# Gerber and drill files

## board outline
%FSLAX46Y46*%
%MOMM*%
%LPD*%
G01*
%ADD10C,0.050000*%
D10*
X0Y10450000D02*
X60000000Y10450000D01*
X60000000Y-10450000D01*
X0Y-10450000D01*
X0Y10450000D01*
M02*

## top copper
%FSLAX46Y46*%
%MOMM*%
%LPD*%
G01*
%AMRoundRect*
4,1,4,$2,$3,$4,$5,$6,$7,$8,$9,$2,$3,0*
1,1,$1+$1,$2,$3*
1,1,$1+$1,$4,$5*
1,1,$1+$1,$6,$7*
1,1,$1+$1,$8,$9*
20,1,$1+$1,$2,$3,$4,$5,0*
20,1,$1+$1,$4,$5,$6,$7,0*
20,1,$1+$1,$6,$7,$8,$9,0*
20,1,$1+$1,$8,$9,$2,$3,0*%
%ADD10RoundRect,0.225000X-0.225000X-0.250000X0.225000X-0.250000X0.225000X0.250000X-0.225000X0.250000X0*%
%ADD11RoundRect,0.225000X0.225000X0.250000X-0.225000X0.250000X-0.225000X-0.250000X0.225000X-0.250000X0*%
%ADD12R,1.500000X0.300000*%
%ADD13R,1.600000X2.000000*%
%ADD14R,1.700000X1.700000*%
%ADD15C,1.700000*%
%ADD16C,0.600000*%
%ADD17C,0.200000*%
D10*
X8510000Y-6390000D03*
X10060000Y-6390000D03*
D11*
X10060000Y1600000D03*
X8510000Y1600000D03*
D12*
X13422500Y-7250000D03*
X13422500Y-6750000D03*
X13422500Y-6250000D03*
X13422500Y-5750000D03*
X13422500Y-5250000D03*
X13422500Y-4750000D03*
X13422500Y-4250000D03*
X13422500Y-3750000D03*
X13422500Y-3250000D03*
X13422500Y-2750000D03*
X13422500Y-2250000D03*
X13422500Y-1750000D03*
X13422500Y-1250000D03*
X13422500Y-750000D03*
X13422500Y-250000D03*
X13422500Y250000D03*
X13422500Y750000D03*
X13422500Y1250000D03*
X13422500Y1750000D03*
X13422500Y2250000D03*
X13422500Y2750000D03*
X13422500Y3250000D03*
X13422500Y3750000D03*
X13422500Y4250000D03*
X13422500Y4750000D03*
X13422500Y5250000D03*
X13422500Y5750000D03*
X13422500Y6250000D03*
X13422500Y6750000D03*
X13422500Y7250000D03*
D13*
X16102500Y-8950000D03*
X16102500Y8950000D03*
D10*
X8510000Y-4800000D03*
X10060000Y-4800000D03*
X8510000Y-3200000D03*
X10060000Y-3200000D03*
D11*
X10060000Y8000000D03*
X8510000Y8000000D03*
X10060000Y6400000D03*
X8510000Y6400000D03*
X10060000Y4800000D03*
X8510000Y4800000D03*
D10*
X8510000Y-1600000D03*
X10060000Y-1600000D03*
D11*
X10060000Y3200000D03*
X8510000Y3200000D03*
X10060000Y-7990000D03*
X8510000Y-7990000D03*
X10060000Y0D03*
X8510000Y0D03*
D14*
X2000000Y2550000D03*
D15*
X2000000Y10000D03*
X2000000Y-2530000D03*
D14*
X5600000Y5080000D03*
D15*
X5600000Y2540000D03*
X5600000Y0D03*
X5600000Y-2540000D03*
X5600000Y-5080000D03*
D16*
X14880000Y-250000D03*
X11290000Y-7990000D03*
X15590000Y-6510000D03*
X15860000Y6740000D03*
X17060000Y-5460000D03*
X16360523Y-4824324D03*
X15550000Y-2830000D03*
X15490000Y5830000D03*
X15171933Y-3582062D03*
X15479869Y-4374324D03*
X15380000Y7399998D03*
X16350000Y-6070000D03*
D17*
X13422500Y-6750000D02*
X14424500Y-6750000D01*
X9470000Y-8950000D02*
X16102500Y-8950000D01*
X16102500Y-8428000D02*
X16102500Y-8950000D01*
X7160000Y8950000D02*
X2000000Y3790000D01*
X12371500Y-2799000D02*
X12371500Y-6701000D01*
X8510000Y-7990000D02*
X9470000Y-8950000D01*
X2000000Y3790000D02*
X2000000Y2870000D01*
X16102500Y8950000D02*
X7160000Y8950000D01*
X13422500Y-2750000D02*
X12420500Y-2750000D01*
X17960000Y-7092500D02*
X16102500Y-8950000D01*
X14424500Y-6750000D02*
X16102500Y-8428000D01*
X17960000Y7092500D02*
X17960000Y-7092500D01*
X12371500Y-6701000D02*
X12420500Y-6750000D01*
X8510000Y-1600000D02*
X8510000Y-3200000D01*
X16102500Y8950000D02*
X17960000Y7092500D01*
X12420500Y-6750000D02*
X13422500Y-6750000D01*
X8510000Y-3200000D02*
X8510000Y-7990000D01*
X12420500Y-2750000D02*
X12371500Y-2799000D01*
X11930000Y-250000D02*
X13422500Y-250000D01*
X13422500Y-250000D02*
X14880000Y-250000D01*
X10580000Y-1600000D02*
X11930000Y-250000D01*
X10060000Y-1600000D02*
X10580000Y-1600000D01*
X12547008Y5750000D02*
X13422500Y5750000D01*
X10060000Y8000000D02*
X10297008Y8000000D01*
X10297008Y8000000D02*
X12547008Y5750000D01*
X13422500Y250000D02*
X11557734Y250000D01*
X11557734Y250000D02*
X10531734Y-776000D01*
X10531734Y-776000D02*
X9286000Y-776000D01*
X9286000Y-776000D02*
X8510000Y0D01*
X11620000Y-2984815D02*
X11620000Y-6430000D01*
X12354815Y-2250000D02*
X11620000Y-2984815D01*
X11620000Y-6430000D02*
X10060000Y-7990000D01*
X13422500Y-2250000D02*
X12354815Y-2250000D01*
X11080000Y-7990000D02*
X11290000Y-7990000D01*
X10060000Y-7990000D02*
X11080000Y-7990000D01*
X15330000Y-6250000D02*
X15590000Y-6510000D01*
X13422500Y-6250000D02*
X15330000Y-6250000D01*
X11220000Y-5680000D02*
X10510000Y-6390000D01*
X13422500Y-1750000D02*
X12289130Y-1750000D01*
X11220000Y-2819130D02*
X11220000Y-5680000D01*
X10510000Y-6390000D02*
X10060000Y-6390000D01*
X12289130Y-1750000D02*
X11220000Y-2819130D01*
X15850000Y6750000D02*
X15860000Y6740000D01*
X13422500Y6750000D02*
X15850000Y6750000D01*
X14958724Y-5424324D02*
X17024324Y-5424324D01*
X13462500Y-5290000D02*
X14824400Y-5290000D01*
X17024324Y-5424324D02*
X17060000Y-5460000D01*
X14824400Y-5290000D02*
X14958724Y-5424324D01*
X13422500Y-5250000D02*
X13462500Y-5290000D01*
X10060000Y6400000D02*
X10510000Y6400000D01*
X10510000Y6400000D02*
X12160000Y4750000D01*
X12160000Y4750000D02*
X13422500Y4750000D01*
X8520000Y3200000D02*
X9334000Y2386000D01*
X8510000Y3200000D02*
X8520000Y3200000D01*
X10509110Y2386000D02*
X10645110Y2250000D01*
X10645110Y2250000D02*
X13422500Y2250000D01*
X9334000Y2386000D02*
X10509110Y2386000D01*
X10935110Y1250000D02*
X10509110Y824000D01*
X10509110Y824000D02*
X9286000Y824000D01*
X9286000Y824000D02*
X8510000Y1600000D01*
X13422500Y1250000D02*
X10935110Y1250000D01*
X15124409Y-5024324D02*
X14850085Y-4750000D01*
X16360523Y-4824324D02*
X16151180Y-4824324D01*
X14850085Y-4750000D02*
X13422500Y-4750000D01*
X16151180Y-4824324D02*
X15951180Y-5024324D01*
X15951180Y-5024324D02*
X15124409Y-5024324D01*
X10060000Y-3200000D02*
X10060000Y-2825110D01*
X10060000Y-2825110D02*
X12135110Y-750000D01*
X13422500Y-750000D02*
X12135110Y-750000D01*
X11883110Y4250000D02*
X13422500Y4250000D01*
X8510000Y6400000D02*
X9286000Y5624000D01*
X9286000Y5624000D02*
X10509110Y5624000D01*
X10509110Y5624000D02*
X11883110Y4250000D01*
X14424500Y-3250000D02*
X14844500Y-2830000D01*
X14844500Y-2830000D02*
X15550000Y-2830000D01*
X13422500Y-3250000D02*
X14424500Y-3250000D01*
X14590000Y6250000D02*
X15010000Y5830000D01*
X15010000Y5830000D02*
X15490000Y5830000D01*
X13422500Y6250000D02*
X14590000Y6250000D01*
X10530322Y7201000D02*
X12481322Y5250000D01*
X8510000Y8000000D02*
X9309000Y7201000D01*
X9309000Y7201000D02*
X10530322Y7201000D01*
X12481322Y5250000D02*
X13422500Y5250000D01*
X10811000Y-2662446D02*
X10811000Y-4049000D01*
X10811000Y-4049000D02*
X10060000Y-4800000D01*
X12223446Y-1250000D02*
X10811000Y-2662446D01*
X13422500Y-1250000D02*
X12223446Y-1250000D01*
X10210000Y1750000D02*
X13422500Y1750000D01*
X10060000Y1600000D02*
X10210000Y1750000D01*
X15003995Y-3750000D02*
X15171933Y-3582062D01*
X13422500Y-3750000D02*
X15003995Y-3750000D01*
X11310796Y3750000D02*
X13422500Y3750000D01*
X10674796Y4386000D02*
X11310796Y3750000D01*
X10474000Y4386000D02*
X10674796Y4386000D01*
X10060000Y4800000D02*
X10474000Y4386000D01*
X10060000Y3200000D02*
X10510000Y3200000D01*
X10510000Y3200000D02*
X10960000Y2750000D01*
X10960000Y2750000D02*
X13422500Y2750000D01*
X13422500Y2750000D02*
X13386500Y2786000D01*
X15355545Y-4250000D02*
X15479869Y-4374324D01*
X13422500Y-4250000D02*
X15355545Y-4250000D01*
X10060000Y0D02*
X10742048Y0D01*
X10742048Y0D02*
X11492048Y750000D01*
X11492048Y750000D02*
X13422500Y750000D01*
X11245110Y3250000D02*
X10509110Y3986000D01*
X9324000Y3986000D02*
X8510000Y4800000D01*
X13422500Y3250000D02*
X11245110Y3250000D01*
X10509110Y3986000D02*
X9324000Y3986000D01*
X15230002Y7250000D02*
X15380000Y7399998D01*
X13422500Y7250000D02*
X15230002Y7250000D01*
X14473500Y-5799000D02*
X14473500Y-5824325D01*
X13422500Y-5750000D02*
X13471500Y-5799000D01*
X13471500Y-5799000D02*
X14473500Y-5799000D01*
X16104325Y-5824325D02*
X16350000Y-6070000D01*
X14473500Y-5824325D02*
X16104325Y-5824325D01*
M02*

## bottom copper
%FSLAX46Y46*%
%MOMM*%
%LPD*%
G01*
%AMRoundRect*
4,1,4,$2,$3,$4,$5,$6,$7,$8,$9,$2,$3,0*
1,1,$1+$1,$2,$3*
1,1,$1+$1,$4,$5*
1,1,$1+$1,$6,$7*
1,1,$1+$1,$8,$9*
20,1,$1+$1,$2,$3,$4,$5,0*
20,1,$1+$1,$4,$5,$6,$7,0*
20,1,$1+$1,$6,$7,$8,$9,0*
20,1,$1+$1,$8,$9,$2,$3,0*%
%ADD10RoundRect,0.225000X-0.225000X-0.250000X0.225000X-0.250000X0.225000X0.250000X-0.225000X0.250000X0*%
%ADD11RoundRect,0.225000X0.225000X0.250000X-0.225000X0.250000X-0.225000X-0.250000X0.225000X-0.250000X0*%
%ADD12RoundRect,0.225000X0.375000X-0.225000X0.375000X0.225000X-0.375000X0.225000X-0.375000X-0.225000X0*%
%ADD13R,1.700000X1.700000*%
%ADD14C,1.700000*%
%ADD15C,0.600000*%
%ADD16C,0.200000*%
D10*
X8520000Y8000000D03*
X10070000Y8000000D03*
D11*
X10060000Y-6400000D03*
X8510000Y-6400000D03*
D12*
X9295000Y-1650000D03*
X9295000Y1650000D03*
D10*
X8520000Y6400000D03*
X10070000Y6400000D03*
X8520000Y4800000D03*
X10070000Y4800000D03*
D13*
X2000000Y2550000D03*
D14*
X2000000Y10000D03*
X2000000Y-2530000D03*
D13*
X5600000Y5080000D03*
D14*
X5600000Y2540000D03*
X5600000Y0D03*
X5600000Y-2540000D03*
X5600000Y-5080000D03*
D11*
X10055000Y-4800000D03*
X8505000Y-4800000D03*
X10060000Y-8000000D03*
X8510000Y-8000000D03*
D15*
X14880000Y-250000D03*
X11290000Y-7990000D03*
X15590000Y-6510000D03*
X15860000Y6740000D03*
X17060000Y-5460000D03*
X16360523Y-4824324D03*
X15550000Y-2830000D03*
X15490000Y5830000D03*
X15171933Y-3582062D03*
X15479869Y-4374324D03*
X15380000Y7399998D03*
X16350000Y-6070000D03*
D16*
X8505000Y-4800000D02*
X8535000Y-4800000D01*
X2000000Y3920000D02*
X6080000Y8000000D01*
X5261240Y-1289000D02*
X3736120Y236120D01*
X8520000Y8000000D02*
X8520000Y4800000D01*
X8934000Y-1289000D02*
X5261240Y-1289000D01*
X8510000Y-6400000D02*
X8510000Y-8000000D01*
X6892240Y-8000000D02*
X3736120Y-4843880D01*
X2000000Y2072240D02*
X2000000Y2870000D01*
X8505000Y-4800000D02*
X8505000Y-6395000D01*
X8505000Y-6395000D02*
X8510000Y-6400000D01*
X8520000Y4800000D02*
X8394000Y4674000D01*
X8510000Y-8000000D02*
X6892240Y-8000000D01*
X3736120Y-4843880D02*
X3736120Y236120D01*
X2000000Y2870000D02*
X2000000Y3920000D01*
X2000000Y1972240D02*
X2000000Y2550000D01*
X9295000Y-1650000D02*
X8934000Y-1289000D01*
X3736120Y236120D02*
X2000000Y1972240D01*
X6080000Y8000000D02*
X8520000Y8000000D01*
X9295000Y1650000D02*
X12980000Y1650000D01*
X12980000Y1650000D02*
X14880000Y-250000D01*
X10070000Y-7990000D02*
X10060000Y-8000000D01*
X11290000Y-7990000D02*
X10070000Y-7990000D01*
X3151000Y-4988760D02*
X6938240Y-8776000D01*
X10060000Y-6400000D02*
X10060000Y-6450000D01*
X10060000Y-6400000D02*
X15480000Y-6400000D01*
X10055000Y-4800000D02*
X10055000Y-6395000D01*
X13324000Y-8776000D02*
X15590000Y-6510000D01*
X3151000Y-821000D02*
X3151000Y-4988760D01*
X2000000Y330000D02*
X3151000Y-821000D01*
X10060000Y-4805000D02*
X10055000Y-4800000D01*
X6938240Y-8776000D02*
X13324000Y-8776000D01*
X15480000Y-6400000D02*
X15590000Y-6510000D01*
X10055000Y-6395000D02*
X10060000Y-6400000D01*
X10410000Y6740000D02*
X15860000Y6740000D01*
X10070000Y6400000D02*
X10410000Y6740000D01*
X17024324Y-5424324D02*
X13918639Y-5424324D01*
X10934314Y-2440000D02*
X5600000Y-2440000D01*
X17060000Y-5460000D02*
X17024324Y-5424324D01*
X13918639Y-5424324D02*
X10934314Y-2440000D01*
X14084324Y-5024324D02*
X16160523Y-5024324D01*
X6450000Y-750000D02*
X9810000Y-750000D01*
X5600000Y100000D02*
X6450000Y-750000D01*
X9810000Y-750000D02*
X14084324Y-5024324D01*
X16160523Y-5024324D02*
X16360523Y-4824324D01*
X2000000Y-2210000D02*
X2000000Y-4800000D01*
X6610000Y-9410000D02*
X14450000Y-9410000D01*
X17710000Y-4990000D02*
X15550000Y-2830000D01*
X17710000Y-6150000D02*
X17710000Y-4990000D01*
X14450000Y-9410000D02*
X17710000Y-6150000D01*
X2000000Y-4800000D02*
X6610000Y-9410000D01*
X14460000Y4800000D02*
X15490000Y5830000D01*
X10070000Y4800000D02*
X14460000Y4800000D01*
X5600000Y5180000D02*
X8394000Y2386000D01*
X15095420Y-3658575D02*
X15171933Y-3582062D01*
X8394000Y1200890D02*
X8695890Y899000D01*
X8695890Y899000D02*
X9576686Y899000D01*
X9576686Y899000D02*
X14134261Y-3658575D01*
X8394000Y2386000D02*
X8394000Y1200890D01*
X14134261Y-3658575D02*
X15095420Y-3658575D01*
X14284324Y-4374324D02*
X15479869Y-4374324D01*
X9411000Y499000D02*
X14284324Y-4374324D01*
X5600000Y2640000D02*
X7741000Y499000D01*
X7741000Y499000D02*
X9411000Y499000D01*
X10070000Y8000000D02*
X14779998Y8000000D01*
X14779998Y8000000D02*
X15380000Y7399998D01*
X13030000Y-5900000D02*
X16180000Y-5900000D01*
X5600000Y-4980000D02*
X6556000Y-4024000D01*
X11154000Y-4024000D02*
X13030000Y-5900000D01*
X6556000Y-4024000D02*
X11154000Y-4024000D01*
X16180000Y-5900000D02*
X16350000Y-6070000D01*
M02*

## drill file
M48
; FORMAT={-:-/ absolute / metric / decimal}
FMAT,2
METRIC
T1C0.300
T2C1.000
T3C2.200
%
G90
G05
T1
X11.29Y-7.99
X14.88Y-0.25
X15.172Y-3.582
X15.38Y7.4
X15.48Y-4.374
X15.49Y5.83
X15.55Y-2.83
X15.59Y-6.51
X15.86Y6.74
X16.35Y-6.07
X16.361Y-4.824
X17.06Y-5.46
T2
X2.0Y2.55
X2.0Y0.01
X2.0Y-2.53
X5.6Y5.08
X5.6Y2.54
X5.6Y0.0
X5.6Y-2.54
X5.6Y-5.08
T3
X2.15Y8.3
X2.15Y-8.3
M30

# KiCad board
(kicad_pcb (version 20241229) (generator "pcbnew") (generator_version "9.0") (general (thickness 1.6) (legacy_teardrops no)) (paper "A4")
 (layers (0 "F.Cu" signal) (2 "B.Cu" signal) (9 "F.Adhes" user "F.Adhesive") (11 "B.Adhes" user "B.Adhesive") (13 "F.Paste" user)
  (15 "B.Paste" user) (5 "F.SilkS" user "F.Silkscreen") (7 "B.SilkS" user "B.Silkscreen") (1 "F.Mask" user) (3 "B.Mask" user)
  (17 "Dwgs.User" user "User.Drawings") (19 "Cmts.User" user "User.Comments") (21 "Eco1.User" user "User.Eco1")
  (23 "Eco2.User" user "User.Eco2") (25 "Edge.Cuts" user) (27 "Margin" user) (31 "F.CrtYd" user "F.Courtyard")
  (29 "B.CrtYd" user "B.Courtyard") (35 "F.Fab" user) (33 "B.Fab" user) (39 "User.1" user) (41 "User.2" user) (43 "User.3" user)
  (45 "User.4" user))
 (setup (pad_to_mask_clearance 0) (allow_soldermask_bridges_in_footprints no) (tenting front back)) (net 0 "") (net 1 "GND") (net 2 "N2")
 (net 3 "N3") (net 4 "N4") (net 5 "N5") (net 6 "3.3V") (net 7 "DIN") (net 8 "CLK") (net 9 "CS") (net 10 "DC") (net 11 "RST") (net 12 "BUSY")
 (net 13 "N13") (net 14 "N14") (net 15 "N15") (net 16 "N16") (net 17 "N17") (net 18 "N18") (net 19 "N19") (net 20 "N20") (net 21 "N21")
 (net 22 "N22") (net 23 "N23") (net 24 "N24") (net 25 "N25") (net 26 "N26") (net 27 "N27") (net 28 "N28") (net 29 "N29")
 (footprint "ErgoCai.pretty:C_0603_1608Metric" (layer "F.Cu") (at 9.285 6.39)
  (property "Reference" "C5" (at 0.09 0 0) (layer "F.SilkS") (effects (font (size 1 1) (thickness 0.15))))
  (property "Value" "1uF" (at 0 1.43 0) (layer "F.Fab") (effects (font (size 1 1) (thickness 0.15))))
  (pad "1" smd roundrect (at -0.775 0) (size 0.9 0.95) (layers "F.Cu" "F.Mask" "F.Paste") (roundrect_rratio 0.25) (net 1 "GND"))
  (pad "2" smd roundrect (at 0.775 0) (size 0.9 0.95) (layers "F.Cu" "F.Mask" "F.Paste") (roundrect_rratio 0.25) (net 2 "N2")))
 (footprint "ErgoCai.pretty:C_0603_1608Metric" (layer "F.Cu") (at 9.285 -1.6 180)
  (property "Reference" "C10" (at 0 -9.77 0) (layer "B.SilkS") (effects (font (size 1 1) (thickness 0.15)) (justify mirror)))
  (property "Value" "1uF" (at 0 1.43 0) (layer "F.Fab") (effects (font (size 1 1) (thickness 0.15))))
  (pad "1" smd roundrect (at -0.775 0 180) (size 0.9 0.95) (layers "F.Cu" "F.Mask" "F.Paste") (roundrect_rratio 0.25) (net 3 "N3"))
  (pad "2" smd roundrect (at 0.775 0 180) (size 0.9 0.95) (layers "F.Cu" "F.Mask" "F.Paste") (roundrect_rratio 0.25) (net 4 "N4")))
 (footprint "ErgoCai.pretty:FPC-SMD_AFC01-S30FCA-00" (layer "F.Cu") (at 14.7625 0 90)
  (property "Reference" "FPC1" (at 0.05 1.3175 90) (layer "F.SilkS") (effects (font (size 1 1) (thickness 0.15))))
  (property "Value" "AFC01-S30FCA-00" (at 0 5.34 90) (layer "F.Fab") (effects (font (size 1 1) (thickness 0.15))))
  (pad "1" smd rect (at -7.25 -1.34 90) (size 0.3 1.5) (layers "F.Cu" "F.Mask" "F.Paste") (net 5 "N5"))
  (pad "2" smd rect (at -6.75 -1.34 90) (size 0.3 1.5) (layers "F.Cu" "F.Mask" "F.Paste") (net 1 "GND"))
  (pad "3" smd rect (at -6.25 -1.34 90) (size 0.3 1.5) (layers "F.Cu" "F.Mask" "F.Paste") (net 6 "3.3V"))
  (pad "4" smd rect (at -5.75 -1.34 90) (size 0.3 1.5) (layers "F.Cu" "F.Mask" "F.Paste") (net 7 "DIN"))
  (pad "5" smd rect (at -5.25 -1.34 90) (size 0.3 1.5) (layers "F.Cu" "F.Mask" "F.Paste") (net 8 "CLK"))
  (pad "6" smd rect (at -4.75 -1.34 90) (size 0.3 1.5) (layers "F.Cu" "F.Mask" "F.Paste") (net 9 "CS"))
  (pad "7" smd rect (at -4.25 -1.34 90) (size 0.3 1.5) (layers "F.Cu" "F.Mask" "F.Paste") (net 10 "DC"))
  (pad "8" smd rect (at -3.75 -1.34 90) (size 0.3 1.5) (layers "F.Cu" "F.Mask" "F.Paste") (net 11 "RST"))
  (pad "9" smd rect (at -3.25 -1.34 90) (size 0.3 1.5) (layers "F.Cu" "F.Mask" "F.Paste") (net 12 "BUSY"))
  (pad "10" smd rect (at -2.75 -1.34 90) (size 0.3 1.5) (layers "F.Cu" "F.Mask" "F.Paste") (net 1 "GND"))
  (pad "11" smd rect (at -2.25 -1.34 90) (size 0.3 1.5) (layers "F.Cu" "F.Mask" "F.Paste") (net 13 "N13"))
  (pad "12" smd rect (at -1.75 -1.34 90) (size 0.3 1.5) (layers "F.Cu" "F.Mask" "F.Paste") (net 2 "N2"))
  (pad "13" smd rect (at -1.25 -1.34 90) (size 0.3 1.5) (layers "F.Cu" "F.Mask" "F.Paste") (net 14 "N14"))
  (pad "14" smd rect (at -0.75 -1.34 90) (size 0.3 1.5) (layers "F.Cu" "F.Mask" "F.Paste") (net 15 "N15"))
  (pad "15" smd rect (at -0.25 -1.34 90) (size 0.3 1.5) (layers "F.Cu" "F.Mask" "F.Paste") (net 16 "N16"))
  (pad "16" smd rect (at 0.25 -1.34 90) (size 0.3 1.5) (layers "F.Cu" "F.Mask" "F.Paste") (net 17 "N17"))
  (pad "17" smd rect (at 0.75 -1.34 90) (size 0.3 1.5) (layers "F.Cu" "F.Mask" "F.Paste") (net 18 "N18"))
  (pad "18" smd rect (at 1.25 -1.34 90) (size 0.3 1.5) (layers "F.Cu" "F.Mask" "F.Paste") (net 4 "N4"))
  (pad "19" smd rect (at 1.75 -1.34 90) (size 0.3 1.5) (layers "F.Cu" "F.Mask" "F.Paste") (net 3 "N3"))
  (pad "20" smd rect (at 2.25 -1.34 90) (size 0.3 1.5) (layers "F.Cu" "F.Mask" "F.Paste") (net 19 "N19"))
  (pad "21" smd rect (at 2.75 -1.34 90) (size 0.3 1.5) (layers "F.Cu" "F.Mask" "F.Paste") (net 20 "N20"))
  (pad "22" smd rect (at 3.25 -1.34 90) (size 0.3 1.5) (layers "F.Cu" "F.Mask" "F.Paste") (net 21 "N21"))
  (pad "23" smd rect (at 3.75 -1.34 90) (size 0.3 1.5) (layers "F.Cu" "F.Mask" "F.Paste") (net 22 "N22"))
  (pad "24" smd rect (at 4.25 -1.34 90) (size 0.3 1.5) (layers "F.Cu" "F.Mask" "F.Paste") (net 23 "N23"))
  (pad "25" smd rect (at 4.75 -1.34 90) (size 0.3 1.5) (layers "F.Cu" "F.Mask" "F.Paste") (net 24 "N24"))
  (pad "26" smd rect (at 5.25 -1.34 90) (size 0.3 1.5) (layers "F.Cu" "F.Mask" "F.Paste") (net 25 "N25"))
  (pad "27" smd rect (at 5.75 -1.34 90) (size 0.3 1.5) (layers "F.Cu" "F.Mask" "F.Paste") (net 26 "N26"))
  (pad "28" smd rect (at 6.25 -1.34 90) (size 0.3 1.5) (layers "F.Cu" "F.Mask" "F.Paste") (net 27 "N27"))
  (pad "29" smd rect (at 6.75 -1.34 90) (size 0.3 1.5) (layers "F.Cu" "F.Mask" "F.Paste") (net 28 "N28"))
  (pad "30" smd rect (at 7.25 -1.34 90) (size 0.3 1.5) (layers "F.Cu" "F.Mask" "F.Paste") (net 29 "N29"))
  (pad "31" smd rect (at -8.95 1.34 90) (size 2 1.6) (layers "F.Cu" "F.Mask" "F.Paste") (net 1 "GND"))
  (pad "32" smd rect (at 8.95 1.34 270) (size 2 1.6) (layers "F.Cu" "F.Mask" "F.Paste") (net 1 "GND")))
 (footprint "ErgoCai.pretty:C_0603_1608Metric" (layer "F.Cu") (at 9.285 4.8)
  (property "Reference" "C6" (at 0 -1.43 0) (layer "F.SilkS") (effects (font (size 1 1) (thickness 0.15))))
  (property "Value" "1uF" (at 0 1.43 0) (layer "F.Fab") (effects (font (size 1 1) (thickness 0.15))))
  (pad "1" smd roundrect (at -0.775 0) (size 0.9 0.95) (layers "F.Cu" "F.Mask" "F.Paste") (roundrect_rratio 0.25) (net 1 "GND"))
  (pad "2" smd roundrect (at 0.775 0) (size 0.9 0.95) (layers "F.Cu" "F.Mask" "F.Paste") (roundrect_rratio 0.25) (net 14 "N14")))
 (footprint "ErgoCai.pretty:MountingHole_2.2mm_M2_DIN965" (layer "F.Cu") (at 2.15 -8.3)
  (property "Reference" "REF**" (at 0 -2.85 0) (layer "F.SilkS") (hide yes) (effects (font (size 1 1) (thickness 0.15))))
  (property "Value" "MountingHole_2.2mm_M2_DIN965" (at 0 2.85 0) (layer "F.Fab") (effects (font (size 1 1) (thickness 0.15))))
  (pad "" np_thru_hole circle (at 0 0) (size 2.2 2.2) (drill 2.2) (layers "*.Cu" "*.Mask")))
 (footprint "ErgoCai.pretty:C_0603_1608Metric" (layer "F.Cu") (at 9.285 3.2)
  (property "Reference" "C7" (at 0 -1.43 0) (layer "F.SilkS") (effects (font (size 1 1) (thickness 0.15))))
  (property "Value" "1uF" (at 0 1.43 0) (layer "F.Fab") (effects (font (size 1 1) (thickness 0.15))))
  (pad "1" smd roundrect (at -0.775 0) (size 0.9 0.95) (layers "F.Cu" "F.Mask" "F.Paste") (roundrect_rratio 0.25) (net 1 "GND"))
  (pad "2" smd roundrect (at 0.775 0) (size 0.9 0.95) (layers "F.Cu" "F.Mask" "F.Paste") (roundrect_rratio 0.25) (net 15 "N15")))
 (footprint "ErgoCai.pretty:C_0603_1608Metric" (layer "F.Cu") (at 9.285 -8 180)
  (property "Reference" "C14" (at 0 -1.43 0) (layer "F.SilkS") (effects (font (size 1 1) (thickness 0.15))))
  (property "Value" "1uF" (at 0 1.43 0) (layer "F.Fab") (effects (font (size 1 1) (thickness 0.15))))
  (pad "1" smd roundrect (at -0.775 0 180) (size 0.9 0.95) (layers "F.Cu" "F.Mask" "F.Paste") (roundrect_rratio 0.25) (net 26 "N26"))
  (pad "2" smd roundrect (at 0.775 0 180) (size 0.9 0.95) (layers "F.Cu" "F.Mask" "F.Paste") (roundrect_rratio 0.25) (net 25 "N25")))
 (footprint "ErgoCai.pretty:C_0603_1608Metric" (layer "F.Cu") (at 9.285 -6.4 180)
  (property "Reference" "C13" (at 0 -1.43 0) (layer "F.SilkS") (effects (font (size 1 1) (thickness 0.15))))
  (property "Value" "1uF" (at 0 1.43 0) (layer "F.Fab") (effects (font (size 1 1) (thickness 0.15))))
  (pad "1" smd roundrect (at -0.775 0 180) (size 0.9 0.95) (layers "F.Cu" "F.Mask" "F.Paste") (roundrect_rratio 0.25) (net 24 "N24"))
  (pad "2" smd roundrect (at 0.775 0 180) (size 0.9 0.95) (layers "F.Cu" "F.Mask" "F.Paste") (roundrect_rratio 0.25) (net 23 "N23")))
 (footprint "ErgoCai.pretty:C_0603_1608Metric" (layer "F.Cu") (at 9.285 -4.8 180)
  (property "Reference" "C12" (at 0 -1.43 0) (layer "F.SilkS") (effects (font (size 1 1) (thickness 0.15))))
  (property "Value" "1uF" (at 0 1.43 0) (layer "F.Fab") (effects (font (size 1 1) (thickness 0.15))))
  (pad "1" smd roundrect (at -0.775 0 180) (size 0.9 0.95) (layers "F.Cu" "F.Mask" "F.Paste") (roundrect_rratio 0.25) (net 22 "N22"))
  (pad "2" smd roundrect (at 0.775 0 180) (size 0.9 0.95) (layers "F.Cu" "F.Mask" "F.Paste") (roundrect_rratio 0.25) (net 21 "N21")))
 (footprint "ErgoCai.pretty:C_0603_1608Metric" (layer "F.Cu") (at 9.285 1.6)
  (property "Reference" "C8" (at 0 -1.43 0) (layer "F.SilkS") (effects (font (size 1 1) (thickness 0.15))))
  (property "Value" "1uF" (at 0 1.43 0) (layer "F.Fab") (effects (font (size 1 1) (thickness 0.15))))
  (pad "1" smd roundrect (at -0.775 0) (size 0.9 0.95) (layers "F.Cu" "F.Mask" "F.Paste") (roundrect_rratio 0.25) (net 1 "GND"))
  (pad "2" smd roundrect (at 0.775 0) (size 0.9 0.95) (layers "F.Cu" "F.Mask" "F.Paste") (roundrect_rratio 0.25) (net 16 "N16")))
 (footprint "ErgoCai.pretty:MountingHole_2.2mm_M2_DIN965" (layer "F.Cu") (at 2.15 8.3)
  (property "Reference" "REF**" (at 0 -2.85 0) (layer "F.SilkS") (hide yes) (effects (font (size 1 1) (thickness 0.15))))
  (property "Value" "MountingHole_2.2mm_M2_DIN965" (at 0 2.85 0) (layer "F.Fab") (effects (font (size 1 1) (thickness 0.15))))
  (pad "" np_thru_hole circle (at 0 0) (size 2.2 2.2) (drill 2.2) (layers "*.Cu" "*.Mask")))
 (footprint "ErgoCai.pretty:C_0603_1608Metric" (layer "F.Cu") (at 9.285 -3.2 180)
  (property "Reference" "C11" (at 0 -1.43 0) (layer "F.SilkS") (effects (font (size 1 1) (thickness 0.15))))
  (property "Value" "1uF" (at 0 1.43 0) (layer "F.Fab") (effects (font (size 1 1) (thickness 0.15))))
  (pad "1" smd roundrect (at -0.775 0 180) (size 0.9 0.95) (layers "F.Cu" "F.Mask" "F.Paste") (roundrect_rratio 0.25) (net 20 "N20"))
  (pad "2" smd roundrect (at 0.775 0 180) (size 0.9 0.95) (layers "F.Cu" "F.Mask" "F.Paste") (roundrect_rratio 0.25) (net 19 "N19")))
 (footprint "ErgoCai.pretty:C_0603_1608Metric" (layer "F.Cu") (at 9.285 7.99 180)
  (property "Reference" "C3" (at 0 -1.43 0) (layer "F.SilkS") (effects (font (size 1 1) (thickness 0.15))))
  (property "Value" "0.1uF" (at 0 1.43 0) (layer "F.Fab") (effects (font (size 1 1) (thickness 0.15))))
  (pad "1" smd roundrect (at -0.775 0 180) (size 0.9 0.95) (layers "F.Cu" "F.Mask" "F.Paste") (roundrect_rratio 0.25) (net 13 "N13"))
  (pad "2" smd roundrect (at 0.775 0 180) (size 0.9 0.95) (layers "F.Cu" "F.Mask" "F.Paste") (roundrect_rratio 0.25) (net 1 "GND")))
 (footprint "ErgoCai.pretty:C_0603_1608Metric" (layer "F.Cu") (at 9.285 0 180)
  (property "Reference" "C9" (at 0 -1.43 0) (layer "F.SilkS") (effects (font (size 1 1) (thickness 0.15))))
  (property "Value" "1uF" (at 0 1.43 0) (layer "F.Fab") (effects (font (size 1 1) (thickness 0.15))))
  (pad "1" smd roundrect (at -0.775 0 180) (size 0.9 0.95) (layers "F.Cu" "F.Mask" "F.Paste") (roundrect_rratio 0.25) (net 18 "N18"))
  (pad "2" smd roundrect (at 0.775 0 180) (size 0.9 0.95) (layers "F.Cu" "F.Mask" "F.Paste") (roundrect_rratio 0.25) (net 17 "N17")))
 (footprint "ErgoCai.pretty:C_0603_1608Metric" (layer "B.Cu") (at 9.295 -8)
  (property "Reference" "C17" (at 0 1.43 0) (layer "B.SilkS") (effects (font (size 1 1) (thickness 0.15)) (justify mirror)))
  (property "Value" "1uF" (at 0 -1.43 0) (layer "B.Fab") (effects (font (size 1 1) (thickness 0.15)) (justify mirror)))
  (pad "1" smd roundrect (at -0.775 0) (size 0.9 0.95) (layers "B.Cu" "B.Mask" "B.Paste") (roundrect_rratio 0.25) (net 1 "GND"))
  (pad "2" smd roundrect (at 0.775 0) (size 0.9 0.95) (layers "B.Cu" "B.Mask" "B.Paste") (roundrect_rratio 0.25) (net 29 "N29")))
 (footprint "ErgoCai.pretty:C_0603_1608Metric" (layer "B.Cu") (at 9.285 6.4 180)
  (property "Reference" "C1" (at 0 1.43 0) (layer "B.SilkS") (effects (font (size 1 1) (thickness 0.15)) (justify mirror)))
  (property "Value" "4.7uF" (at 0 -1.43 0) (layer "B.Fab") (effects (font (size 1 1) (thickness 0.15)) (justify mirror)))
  (pad "1" smd roundrect (at -0.775 0 180) (size 0.9 0.95) (layers "B.Cu" "B.Mask" "B.Paste") (roundrect_rratio 0.25) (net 6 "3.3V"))
  (pad "2" smd roundrect (at 0.775 0 180) (size 0.9 0.95) (layers "B.Cu" "B.Mask" "B.Paste") (roundrect_rratio 0.25) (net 1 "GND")))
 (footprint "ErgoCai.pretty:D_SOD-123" (layer "B.Cu") (at 9.295 0 90)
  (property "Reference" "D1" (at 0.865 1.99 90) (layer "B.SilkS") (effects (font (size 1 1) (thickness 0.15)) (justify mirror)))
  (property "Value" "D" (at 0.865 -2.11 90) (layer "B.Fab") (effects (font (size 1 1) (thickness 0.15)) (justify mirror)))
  (pad "1" smd roundrect (at -1.65 0 90) (size 0.9 1.2) (layers "B.Cu" "B.Mask" "B.Paste") (roundrect_rratio 0.25) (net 1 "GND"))
  (pad "2" smd roundrect (at 1.65 0 90) (size 0.9 1.2) (layers "B.Cu" "B.Mask" "B.Paste") (roundrect_rratio 0.25) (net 16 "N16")))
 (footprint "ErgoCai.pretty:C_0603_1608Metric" (layer "B.Cu") (at 9.295 -6.4)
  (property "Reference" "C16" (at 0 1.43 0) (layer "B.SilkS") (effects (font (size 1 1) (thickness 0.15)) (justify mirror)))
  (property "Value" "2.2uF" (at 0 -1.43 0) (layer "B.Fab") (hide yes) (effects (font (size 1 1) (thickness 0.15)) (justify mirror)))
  (pad "1" smd roundrect (at -0.775 0) (size 0.9 0.95) (layers "B.Cu" "B.Mask" "B.Paste") (roundrect_rratio 0.25) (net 1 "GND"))
  (pad "2" smd roundrect (at 0.775 0) (size 0.9 0.95) (layers "B.Cu" "B.Mask" "B.Paste") (roundrect_rratio 0.25) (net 28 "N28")))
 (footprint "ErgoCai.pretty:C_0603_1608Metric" (layer "B.Cu") (at 9.295 -4.8)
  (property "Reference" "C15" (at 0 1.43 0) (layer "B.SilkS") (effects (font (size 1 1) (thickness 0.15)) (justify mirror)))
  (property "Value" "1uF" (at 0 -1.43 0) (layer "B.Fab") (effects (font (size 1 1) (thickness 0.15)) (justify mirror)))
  (pad "1" smd roundrect (at -0.775 0) (size 0.9 0.95) (layers "B.Cu" "B.Mask" "B.Paste") (roundrect_rratio 0.25) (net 1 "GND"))
  (pad "2" smd roundrect (at 0.775 0) (size 0.9 0.95) (layers "B.Cu" "B.Mask" "B.Paste") (roundrect_rratio 0.25) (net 27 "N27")))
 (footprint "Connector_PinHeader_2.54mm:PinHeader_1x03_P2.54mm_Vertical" (layer "B.Cu") (at 2 -2.55 180)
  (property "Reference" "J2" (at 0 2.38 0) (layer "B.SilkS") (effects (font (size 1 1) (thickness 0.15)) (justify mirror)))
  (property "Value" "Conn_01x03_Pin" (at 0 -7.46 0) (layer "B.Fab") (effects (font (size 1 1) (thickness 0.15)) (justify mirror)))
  (pad "1" thru_hole rect (at 0 0 180) (size 1.7 1.7) (drill 1) (layers "*.Cu" "*.Mask") (remove_unused_layers no) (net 1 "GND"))
  (pad "2" thru_hole circle (at 0 -2.54 180) (size 1.7 1.7) (drill 1) (layers "*.Cu" "*.Mask") (remove_unused_layers no) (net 6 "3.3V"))
  (pad "3" thru_hole circle (at 0 -5.08 180) (size 1.7 1.7) (drill 1) (layers "*.Cu" "*.Mask") (remove_unused_layers no) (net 12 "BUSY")))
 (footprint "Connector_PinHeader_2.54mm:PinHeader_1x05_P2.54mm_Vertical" (layer "B.Cu") (at 5.6 -5.08 180)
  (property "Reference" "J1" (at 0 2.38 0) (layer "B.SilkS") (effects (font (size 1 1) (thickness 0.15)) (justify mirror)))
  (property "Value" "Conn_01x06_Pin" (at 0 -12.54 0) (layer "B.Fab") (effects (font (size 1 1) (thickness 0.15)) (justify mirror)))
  (pad "1" thru_hole rect (at 0 0 180) (size 1.7 1.7) (drill 1) (layers "*.Cu" "*.Mask") (remove_unused_layers no) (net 11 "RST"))
  (pad "2" thru_hole circle (at 0 -2.54 180) (size 1.7 1.7) (drill 1) (layers "*.Cu" "*.Mask") (remove_unused_layers no) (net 10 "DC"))
  (pad "3" thru_hole circle (at 0 -5.08 180) (size 1.7 1.7) (drill 1) (layers "*.Cu" "*.Mask") (remove_unused_layers no) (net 9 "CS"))
  (pad "4" thru_hole circle (at 0 -7.62 180) (size 1.7 1.7) (drill 1) (layers "*.Cu" "*.Mask") (remove_unused_layers no) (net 8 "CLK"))
  (pad "5" thru_hole circle (at 0 -10.16 180) (size 1.7 1.7) (drill 1) (layers "*.Cu" "*.Mask") (remove_unused_layers no) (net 7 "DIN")))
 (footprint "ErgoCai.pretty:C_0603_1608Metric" (layer "B.Cu") (at 9.28 4.8 180)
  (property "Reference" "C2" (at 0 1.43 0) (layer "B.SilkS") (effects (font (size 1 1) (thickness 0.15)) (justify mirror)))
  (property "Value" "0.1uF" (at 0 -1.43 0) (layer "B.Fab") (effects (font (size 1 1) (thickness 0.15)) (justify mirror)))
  (pad "1" smd roundrect (at -0.775 0 180) (size 0.9 0.95) (layers "B.Cu" "B.Mask" "B.Paste") (roundrect_rratio 0.25) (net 6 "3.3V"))
  (pad "2" smd roundrect (at 0.775 0 180) (size 0.9 0.95) (layers "B.Cu" "B.Mask" "B.Paste") (roundrect_rratio 0.25) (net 1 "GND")))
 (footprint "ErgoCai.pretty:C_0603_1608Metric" (layer "B.Cu") (at 9.285 8 180)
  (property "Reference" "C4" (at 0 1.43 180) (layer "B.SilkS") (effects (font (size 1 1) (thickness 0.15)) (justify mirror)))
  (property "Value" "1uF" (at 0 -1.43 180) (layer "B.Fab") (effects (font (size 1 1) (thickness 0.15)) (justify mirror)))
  (pad "1" smd roundrect (at -0.775 0 180) (size 0.9 0.95) (layers "B.Cu" "B.Mask" "B.Paste") (roundrect_rratio 0.25) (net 13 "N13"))
  (pad "2" smd roundrect (at 0.775 0 180) (size 0.9 0.95) (layers "B.Cu" "B.Mask" "B.Paste") (roundrect_rratio 0.25) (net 1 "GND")))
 (gr_rect (start 0 -10.45) (end 60 10.45) (stroke (width 0.05) (type solid)) (fill no) (layer "Edge.Cuts"))
 (segment (start 13.4225 6.75) (end 14.4245 6.75) (width 0.2) (layer "F.Cu") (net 1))
 (segment (start 9.47 8.95) (end 16.1025 8.95) (width 0.2) (layer "F.Cu") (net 1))
 (segment (start 16.1025 8.428) (end 16.1025 8.95) (width 0.2) (layer "F.Cu") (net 1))
 (segment (start 7.16 -8.95) (end 2 -3.79) (width 0.2) (layer "F.Cu") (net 1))
 (segment (start 12.3715 2.799) (end 12.3715 6.701) (width 0.2) (layer "F.Cu") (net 1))
 (segment (start 8.51 7.99) (end 9.47 8.95) (width 0.2) (layer "F.Cu") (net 1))
 (segment (start 2 -3.79) (end 2 -2.87) (width 0.2) (layer "F.Cu") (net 1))
 (segment (start 16.1025 -8.95) (end 7.16 -8.95) (width 0.2) (layer "F.Cu") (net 1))
 (segment (start 13.4225 2.75) (end 12.4205 2.75) (width 0.2) (layer "F.Cu") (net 1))
 (segment (start 17.96 7.0925) (end 16.1025 8.95) (width 0.2) (layer "F.Cu") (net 1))
 (segment (start 14.4245 6.75) (end 16.1025 8.428) (width 0.2) (layer "F.Cu") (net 1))
 (segment (start 17.96 -7.0925) (end 17.96 7.0925) (width 0.2) (layer "F.Cu") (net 1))
 (segment (start 12.3715 6.701) (end 12.4205 6.75) (width 0.2) (layer "F.Cu") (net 1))
 (segment (start 8.51 1.6) (end 8.51 3.2) (width 0.2) (layer "F.Cu") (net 1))
 (segment (start 16.1025 -8.95) (end 17.96 -7.0925) (width 0.2) (layer "F.Cu") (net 1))
 (segment (start 12.4205 6.75) (end 13.4225 6.75) (width 0.2) (layer "F.Cu") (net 1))
 (segment (start 8.51 3.2) (end 8.51 7.99) (width 0.2) (layer "F.Cu") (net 1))
 (segment (start 12.4205 2.75) (end 12.3715 2.799) (width 0.2) (layer "F.Cu") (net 1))
 (segment (start 8.505 4.8) (end 8.535 4.8) (width 0.2) (layer "B.Cu") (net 1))
 (segment (start 2 -3.92) (end 6.08 -8) (width 0.2) (layer "B.Cu") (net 1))
 (segment (start 5.26124 1.289) (end 3.73612 -0.23612) (width 0.2) (layer "B.Cu") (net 1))
 (segment (start 8.52 -8) (end 8.52 -4.8) (width 0.2) (layer "B.Cu") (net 1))
 (segment (start 8.934 1.289) (end 5.26124 1.289) (width 0.2) (layer "B.Cu") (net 1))
 (segment (start 8.51 6.4) (end 8.51 8) (width 0.2) (layer "B.Cu") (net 1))
 (segment (start 6.89224 8) (end 3.73612 4.84388) (width 0.2) (layer "B.Cu") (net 1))
 (segment (start 2 -2.07224) (end 2 -2.87) (width 0.2) (layer "B.Cu") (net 1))
 (segment (start 8.505 4.8) (end 8.505 6.395) (width 0.2) (layer "B.Cu") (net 1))
 (segment (start 8.505 6.395) (end 8.51 6.4) (width 0.2) (layer "B.Cu") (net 1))
 (segment (start 8.52 -4.8) (end 8.394 -4.674) (width 0.2) (layer "B.Cu") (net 1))
 (segment (start 8.51 8) (end 6.89224 8) (width 0.2) (layer "B.Cu") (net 1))
 (segment (start 3.73612 4.84388) (end 3.73612 -0.23612) (width 0.2) (layer "B.Cu") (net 1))
 (segment (start 2 -2.87) (end 2 -3.92) (width 0.2) (layer "B.Cu") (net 1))
 (segment (start 2 -1.97224) (end 2 -2.55) (width 0.2) (layer "B.Cu") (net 1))
 (segment (start 9.295 1.65) (end 8.934 1.289) (width 0.2) (layer "B.Cu") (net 1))
 (segment (start 3.73612 -0.23612) (end 2 -1.97224) (width 0.2) (layer "B.Cu") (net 1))
 (segment (start 6.08 -8) (end 8.52 -8) (width 0.2) (layer "B.Cu") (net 1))
 (segment (start 11.93 0.25) (end 13.4225 0.25) (width 0.2) (layer "F.Cu") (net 16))
 (segment (start 13.4225 0.25) (end 14.88 0.25) (width 0.2) (layer "F.Cu") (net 16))
 (segment (start 10.58 1.6) (end 11.93 0.25) (width 0.2) (layer "F.Cu") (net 16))
 (segment (start 10.06 1.6) (end 10.58 1.6) (width 0.2) (layer "F.Cu") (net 16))
 (via (at 14.88 0.25) (size 0.6) (drill 0.3) (layers "F.Cu" "B.Cu") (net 16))
 (segment (start 9.295 -1.65) (end 12.98 -1.65) (width 0.2) (layer "B.Cu") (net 16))
 (segment (start 12.98 -1.65) (end 14.88 0.25) (width 0.2) (layer "B.Cu") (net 16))
 (segment (start 12.547008 -5.75) (end 13.4225 -5.75) (width 0.2) (layer "F.Cu") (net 26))
 (segment (start 10.06 -8) (end 10.297008 -8) (width 0.2) (layer "F.Cu") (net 26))
 (segment (start 10.297008 -8) (end 12.547008 -5.75) (width 0.2) (layer "F.Cu") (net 26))
 (segment (start 13.4225 -0.25) (end 11.557734 -0.25) (width 0.2) (layer "F.Cu") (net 17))
 (segment (start 11.557734 -0.25) (end 10.531734 0.776) (width 0.2) (layer "F.Cu") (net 17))
 (segment (start 10.531734 0.776) (end 9.286 0.776) (width 0.2) (layer "F.Cu") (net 17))
 (segment (start 9.286 0.776) (end 8.51 0) (width 0.2) (layer "F.Cu") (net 17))
 (segment (start 11.62 2.984815) (end 11.62 6.43) (width 0.2) (layer "F.Cu") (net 13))
 (segment (start 12.354815 2.25) (end 11.62 2.984815) (width 0.2) (layer "F.Cu") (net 13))
 (segment (start 11.62 6.43) (end 10.06 7.99) (width 0.2) (layer "F.Cu") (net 13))
 (segment (start 13.4225 2.25) (end 12.354815 2.25) (width 0.2) (layer "F.Cu") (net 13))
 (segment (start 11.08 7.99) (end 11.29 7.99) (width 0.2) (layer "F.Cu") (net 13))
 (segment (start 10.06 7.99) (end 11.08 7.99) (width 0.2) (layer "F.Cu") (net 13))
 (via (at 11.29 7.99) (size 0.6) (drill 0.3) (layers "F.Cu" "B.Cu") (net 13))
 (segment (start 10.07 7.99) (end 10.06 8) (width 0.2) (layer "B.Cu") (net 13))
 (segment (start 11.29 7.99) (end 10.07 7.99) (width 0.2) (layer "B.Cu") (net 13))
 (segment (start 15.33 6.25) (end 15.59 6.51) (width 0.2) (layer "F.Cu") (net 6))
 (segment (start 13.4225 6.25) (end 15.33 6.25) (width 0.2) (layer "F.Cu") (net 6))
 (via (at 15.59 6.51) (size 0.6) (drill 0.3) (layers "F.Cu" "B.Cu") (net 6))
 (segment (start 3.151 4.98876) (end 6.93824 8.776) (width 0.2) (layer "B.Cu") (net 6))
 (segment (start 10.06 6.4) (end 10.06 6.45) (width 0.2) (layer "B.Cu") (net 6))
 (segment (start 10.06 6.4) (end 15.48 6.4) (width 0.2) (layer "B.Cu") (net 6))
 (segment (start 10.055 4.8) (end 10.055 6.395) (width 0.2) (layer "B.Cu") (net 6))
 (segment (start 13.324 8.776) (end 15.59 6.51) (width 0.2) (layer "B.Cu") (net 6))
 (segment (start 3.151 0.821) (end 3.151 4.98876) (width 0.2) (layer "B.Cu") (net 6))
 (segment (start 2 -0.33) (end 3.151 0.821) (width 0.2) (layer "B.Cu") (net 6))
 (segment (start 10.06 4.805) (end 10.055 4.8) (width 0.2) (layer "B.Cu") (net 6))
 (segment (start 6.93824 8.776) (end 13.324 8.776) (width 0.2) (layer "B.Cu") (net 6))
 (segment (start 15.48 6.4) (end 15.59 6.51) (width 0.2) (layer "B.Cu") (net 6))
 (segment (start 10.055 6.395) (end 10.06 6.4) (width 0.2) (layer "B.Cu") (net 6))
 (segment (start 11.22 5.68) (end 10.51 6.39) (width 0.2) (layer "F.Cu") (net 2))
 (segment (start 13.4225 1.75) (end 12.28913 1.75) (width 0.2) (layer "F.Cu") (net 2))
 (segment (start 11.22 2.81913) (end 11.22 5.68) (width 0.2) (layer "F.Cu") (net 2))
 (segment (start 10.51 6.39) (end 10.06 6.39) (width 0.2) (layer "F.Cu") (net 2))
 (segment (start 12.28913 1.75) (end 11.22 2.81913) (width 0.2) (layer "F.Cu") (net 2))
 (segment (start 15.85 -6.75) (end 15.86 -6.74) (width 0.2) (layer "F.Cu") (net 28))
 (segment (start 13.4225 -6.75) (end 15.85 -6.75) (width 0.2) (layer "F.Cu") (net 28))
 (via (at 15.86 -6.74) (size 0.6) (drill 0.3) (layers "F.Cu" "B.Cu") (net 28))
 (segment (start 10.41 -6.74) (end 15.86 -6.74) (width 0.2) (layer "B.Cu") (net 28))
 (segment (start 10.07 -6.4) (end 10.41 -6.74) (width 0.2) (layer "B.Cu") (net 28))
 (segment (start 14.958724 5.424324) (end 17.024324 5.424324) (width 0.2) (layer "F.Cu") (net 8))
 (segment (start 13.4625 5.29) (end 14.8244 5.29) (width 0.2) (layer "F.Cu") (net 8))
 (segment (start 17.024324 5.424324) (end 17.06 5.46) (width 0.2) (layer "F.Cu") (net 8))
 (segment (start 14.8244 5.29) (end 14.958724 5.424324) (width 0.2) (layer "F.Cu") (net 8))
 (segment (start 13.4225 5.25) (end 13.4625 5.29) (width 0.2) (layer "F.Cu") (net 8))
 (via (at 17.06 5.46) (size 0.6) (drill 0.3) (layers "F.Cu" "B.Cu") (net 8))
 (segment (start 17.024324 5.424324) (end 13.918639 5.424324) (width 0.2) (layer "B.Cu") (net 8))
 (segment (start 10.934314 2.44) (end 5.6 2.44) (width 0.2) (layer "B.Cu") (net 8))
 (segment (start 17.06 5.46) (end 17.024324 5.424324) (width 0.2) (layer "B.Cu") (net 8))
 (segment (start 13.918639 5.424324) (end 10.934314 2.44) (width 0.2) (layer "B.Cu") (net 8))
 (segment (start 10.06 -6.4) (end 10.51 -6.4) (width 0.2) (layer "F.Cu") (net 24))
 (segment (start 10.51 -6.4) (end 12.16 -4.75) (width 0.2) (layer "F.Cu") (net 24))
 (segment (start 12.16 -4.75) (end 13.4225 -4.75) (width 0.2) (layer "F.Cu") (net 24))
 (segment (start 8.52 -3.2) (end 9.334 -2.386) (width 0.2) (layer "F.Cu") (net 19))
 (segment (start 8.51 -3.2) (end 8.52 -3.2) (width 0.2) (layer "F.Cu") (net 19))
 (segment (start 10.50911 -2.386) (end 10.64511 -2.25) (width 0.2) (layer "F.Cu") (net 19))
 (segment (start 10.64511 -2.25) (end 13.4225 -2.25) (width 0.2) (layer "F.Cu") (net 19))
 (segment (start 9.334 -2.386) (end 10.50911 -2.386) (width 0.2) (layer "F.Cu") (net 19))
 (segment (start 10.93511 -1.25) (end 10.50911 -0.824) (width 0.2) (layer "F.Cu") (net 4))
 (segment (start 10.50911 -0.824) (end 9.286 -0.824) (width 0.2) (layer "F.Cu") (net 4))
 (segment (start 9.286 -0.824) (end 8.51 -1.6) (width 0.2) (layer "F.Cu") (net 4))
 (segment (start 13.4225 -1.25) (end 10.93511 -1.25) (width 0.2) (layer "F.Cu") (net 4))
 (segment (start 15.124409 5.024324) (end 14.850085 4.75) (width 0.2) (layer "F.Cu") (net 9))
 (segment (start 16.360523 4.824324) (end 16.15118 4.824324) (width 0.2) (layer "F.Cu") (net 9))
 (segment (start 14.850085 4.75) (end 13.4225 4.75) (width 0.2) (layer "F.Cu") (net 9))
 (segment (start 16.15118 4.824324) (end 15.95118 5.024324) (width 0.2) (layer "F.Cu") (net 9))
 (segment (start 15.95118 5.024324) (end 15.124409 5.024324) (width 0.2) (layer "F.Cu") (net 9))
 (via (at 16.360523 4.824324) (size 0.6) (drill 0.3) (layers "F.Cu" "B.Cu") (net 9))
 (segment (start 14.084324 5.024324) (end 16.160523 5.024324) (width 0.2) (layer "B.Cu") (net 9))
 (segment (start 6.45 0.75) (end 9.81 0.75) (width 0.2) (layer "B.Cu") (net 9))
 (segment (start 5.6 -0.1) (end 6.45 0.75) (width 0.2) (layer "B.Cu") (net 9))
 (segment (start 9.81 0.75) (end 14.084324 5.024324) (width 0.2) (layer "B.Cu") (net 9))
 (segment (start 16.160523 5.024324) (end 16.360523 4.824324) (width 0.2) (layer "B.Cu") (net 9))
 (segment (start 10.06 3.2) (end 10.06 2.82511) (width 0.2) (layer "F.Cu") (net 15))
 (segment (start 10.06 2.82511) (end 12.13511 0.75) (width 0.2) (layer "F.Cu") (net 15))
 (segment (start 13.4225 0.75) (end 12.13511 0.75) (width 0.2) (layer "F.Cu") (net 15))
 (segment (start 11.88311 -4.25) (end 13.4225 -4.25) (width 0.2) (layer "F.Cu") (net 23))
 (segment (start 8.51 -6.4) (end 9.286 -5.624) (width 0.2) (layer "F.Cu") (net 23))
 (segment (start 9.286 -5.624) (end 10.50911 -5.624) (width 0.2) (layer "F.Cu") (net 23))
 (segment (start 10.50911 -5.624) (end 11.88311 -4.25) (width 0.2) (layer "F.Cu") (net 23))
 (segment (start 14.4245 3.25) (end 14.8445 2.83) (width 0.2) (layer "F.Cu") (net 12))
 (segment (start 14.8445 2.83) (end 15.55 2.83) (width 0.2) (layer "F.Cu") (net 12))
 (segment (start 13.4225 3.25) (end 14.4245 3.25) (width 0.2) (layer "F.Cu") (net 12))
 (via (at 15.55 2.83) (size 0.6) (drill 0.3) (layers "F.Cu" "B.Cu") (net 12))
 (segment (start 2 2.21) (end 2 4.8) (width 0.2) (layer "B.Cu") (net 12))
 (segment (start 6.61 9.41) (end 14.45 9.41) (width 0.2) (layer "B.Cu") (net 12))
 (segment (start 17.71 4.99) (end 15.55 2.83) (width 0.2) (layer "B.Cu") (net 12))
 (segment (start 17.71 6.15) (end 17.71 4.99) (width 0.2) (layer "B.Cu") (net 12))
 (segment (start 14.45 9.41) (end 17.71 6.15) (width 0.2) (layer "B.Cu") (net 12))
 (segment (start 2 4.8) (end 6.61 9.41) (width 0.2) (layer "B.Cu") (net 12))
 (segment (start 14.59 -6.25) (end 15.01 -5.83) (width 0.2) (layer "F.Cu") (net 27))
 (segment (start 15.01 -5.83) (end 15.49 -5.83) (width 0.2) (layer "F.Cu") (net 27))
 (segment (start 13.4225 -6.25) (end 14.59 -6.25) (width 0.2) (layer "F.Cu") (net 27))
 (via (at 15.49 -5.83) (size 0.6) (drill 0.3) (layers "F.Cu" "B.Cu") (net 27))
 (segment (start 14.46 -4.8) (end 15.49 -5.83) (width 0.2) (layer "B.Cu") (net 27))
 (segment (start 10.07 -4.8) (end 14.46 -4.8) (width 0.2) (layer "B.Cu") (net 27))
 (segment (start 10.530322 -7.201) (end 12.481322 -5.25) (width 0.2) (layer "F.Cu") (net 25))
 (segment (start 8.51 -8) (end 9.309 -7.201) (width 0.2) (layer "F.Cu") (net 25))
 (segment (start 9.309 -7.201) (end 10.530322 -7.201) (width 0.2) (layer "F.Cu") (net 25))
 (segment (start 12.481322 -5.25) (end 13.4225 -5.25) (width 0.2) (layer "F.Cu") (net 25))
 (segment (start 10.811 2.662446) (end 10.811 4.049) (width 0.2) (layer "F.Cu") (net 14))
 (segment (start 10.811 4.049) (end 10.06 4.8) (width 0.2) (layer "F.Cu") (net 14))
 (segment (start 12.223446 1.25) (end 10.811 2.662446) (width 0.2) (layer "F.Cu") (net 14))
 (segment (start 13.4225 1.25) (end 12.223446 1.25) (width 0.2) (layer "F.Cu") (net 14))
 (segment (start 10.21 -1.75) (end 13.4225 -1.75) (width 0.2) (layer "F.Cu") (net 3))
 (segment (start 10.06 -1.6) (end 10.21 -1.75) (width 0.2) (layer "F.Cu") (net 3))
 (segment (start 15.003995 3.75) (end 15.171933 3.582062) (width 0.2) (layer "F.Cu") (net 11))
 (segment (start 13.4225 3.75) (end 15.003995 3.75) (width 0.2) (layer "F.Cu") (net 11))
 (via (at 15.171933 3.582062) (size 0.6) (drill 0.3) (layers "F.Cu" "B.Cu") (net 11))
 (segment (start 5.6 -5.18) (end 8.394 -2.386) (width 0.2) (layer "B.Cu") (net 11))
 (segment (start 15.09542 3.658575) (end 15.171933 3.582062) (width 0.2) (layer "B.Cu") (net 11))
 (segment (start 8.394 -1.20089) (end 8.69589 -0.899) (width 0.2) (layer "B.Cu") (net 11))
 (segment (start 8.69589 -0.899) (end 9.576686 -0.899) (width 0.2) (layer "B.Cu") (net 11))
 (segment (start 9.576686 -0.899) (end 14.134261 3.658575) (width 0.2) (layer "B.Cu") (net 11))
 (segment (start 8.394 -2.386) (end 8.394 -1.20089) (width 0.2) (layer "B.Cu") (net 11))
 (segment (start 14.134261 3.658575) (end 15.09542 3.658575) (width 0.2) (layer "B.Cu") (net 11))
 (segment (start 11.310796 -3.75) (end 13.4225 -3.75) (width 0.2) (layer "F.Cu") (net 22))
 (segment (start 10.674796 -4.386) (end 11.310796 -3.75) (width 0.2) (layer "F.Cu") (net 22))
 (segment (start 10.474 -4.386) (end 10.674796 -4.386) (width 0.2) (layer "F.Cu") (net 22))
 (segment (start 10.06 -4.8) (end 10.474 -4.386) (width 0.2) (layer "F.Cu") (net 22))
 (segment (start 10.06 -3.2) (end 10.51 -3.2) (width 0.2) (layer "F.Cu") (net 20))
 (segment (start 10.51 -3.2) (end 10.96 -2.75) (width 0.2) (layer "F.Cu") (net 20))
 (segment (start 10.96 -2.75) (end 13.4225 -2.75) (width 0.2) (layer "F.Cu") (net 20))
 (segment (start 13.4225 -2.75) (end 13.3865 -2.786) (width 0.2) (layer "F.Cu") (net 20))
 (segment (start 15.355545 4.25) (end 15.479869 4.374324) (width 0.2) (layer "F.Cu") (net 10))
 (segment (start 13.4225 4.25) (end 15.355545 4.25) (width 0.2) (layer "F.Cu") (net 10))
 (via (at 15.479869 4.374324) (size 0.6) (drill 0.3) (layers "F.Cu" "B.Cu") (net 10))
 (segment (start 14.284324 4.374324) (end 15.479869 4.374324) (width 0.2) (layer "B.Cu") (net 10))
 (segment (start 9.411 -0.499) (end 14.284324 4.374324) (width 0.2) (layer "B.Cu") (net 10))
 (segment (start 5.6 -2.64) (end 7.741 -0.499) (width 0.2) (layer "B.Cu") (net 10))
 (segment (start 7.741 -0.499) (end 9.411 -0.499) (width 0.2) (layer "B.Cu") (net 10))
 (segment (start 10.06 0) (end 10.742048 0) (width 0.2) (layer "F.Cu") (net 18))
 (segment (start 10.742048 0) (end 11.492048 -0.75) (width 0.2) (layer "F.Cu") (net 18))
 (segment (start 11.492048 -0.75) (end 13.4225 -0.75) (width 0.2) (layer "F.Cu") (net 18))
 (segment (start 11.24511 -3.25) (end 10.50911 -3.986) (width 0.2) (layer "F.Cu") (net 21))
 (segment (start 9.324 -3.986) (end 8.51 -4.8) (width 0.2) (layer "F.Cu") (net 21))
 (segment (start 13.4225 -3.25) (end 11.24511 -3.25) (width 0.2) (layer "F.Cu") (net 21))
 (segment (start 10.50911 -3.986) (end 9.324 -3.986) (width 0.2) (layer "F.Cu") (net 21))
 (segment (start 15.230002 -7.25) (end 15.38 -7.399998) (width 0.2) (layer "F.Cu") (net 29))
 (segment (start 13.4225 -7.25) (end 15.230002 -7.25) (width 0.2) (layer "F.Cu") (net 29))
 (via (at 15.38 -7.399998) (size 0.6) (drill 0.3) (layers "F.Cu" "B.Cu") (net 29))
 (segment (start 10.07 -8) (end 14.779998 -8) (width 0.2) (layer "B.Cu") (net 29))
 (segment (start 14.779998 -8) (end 15.38 -7.399998) (width 0.2) (layer "B.Cu") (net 29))
 (segment (start 14.4735 5.799) (end 14.4735 5.824325) (width 0.2) (layer "F.Cu") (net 7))
 (segment (start 13.4225 5.75) (end 13.4715 5.799) (width 0.2) (layer "F.Cu") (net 7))
 (segment (start 13.4715 5.799) (end 14.4735 5.799) (width 0.2) (layer "F.Cu") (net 7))
 (segment (start 16.104325 5.824325) (end 16.35 6.07) (width 0.2) (layer "F.Cu") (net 7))
 (segment (start 14.4735 5.824325) (end 16.104325 5.824325) (width 0.2) (layer "F.Cu") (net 7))
 (via (at 16.35 6.07) (size 0.6) (drill 0.3) (layers "F.Cu" "B.Cu") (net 7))
 (segment (start 13.03 5.9) (end 16.18 5.9) (width 0.2) (layer "B.Cu") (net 7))
 (segment (start 5.6 4.98) (end 6.556 4.024) (width 0.2) (layer "B.Cu") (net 7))
 (segment (start 11.154 4.024) (end 13.03 5.9) (width 0.2) (layer "B.Cu") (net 7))
 (segment (start 6.556 4.024) (end 11.154 4.024) (width 0.2) (layer "B.Cu") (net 7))
 (segment (start 16.18 5.9) (end 16.35 6.07) (width 0.2) (layer "B.Cu") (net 7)))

